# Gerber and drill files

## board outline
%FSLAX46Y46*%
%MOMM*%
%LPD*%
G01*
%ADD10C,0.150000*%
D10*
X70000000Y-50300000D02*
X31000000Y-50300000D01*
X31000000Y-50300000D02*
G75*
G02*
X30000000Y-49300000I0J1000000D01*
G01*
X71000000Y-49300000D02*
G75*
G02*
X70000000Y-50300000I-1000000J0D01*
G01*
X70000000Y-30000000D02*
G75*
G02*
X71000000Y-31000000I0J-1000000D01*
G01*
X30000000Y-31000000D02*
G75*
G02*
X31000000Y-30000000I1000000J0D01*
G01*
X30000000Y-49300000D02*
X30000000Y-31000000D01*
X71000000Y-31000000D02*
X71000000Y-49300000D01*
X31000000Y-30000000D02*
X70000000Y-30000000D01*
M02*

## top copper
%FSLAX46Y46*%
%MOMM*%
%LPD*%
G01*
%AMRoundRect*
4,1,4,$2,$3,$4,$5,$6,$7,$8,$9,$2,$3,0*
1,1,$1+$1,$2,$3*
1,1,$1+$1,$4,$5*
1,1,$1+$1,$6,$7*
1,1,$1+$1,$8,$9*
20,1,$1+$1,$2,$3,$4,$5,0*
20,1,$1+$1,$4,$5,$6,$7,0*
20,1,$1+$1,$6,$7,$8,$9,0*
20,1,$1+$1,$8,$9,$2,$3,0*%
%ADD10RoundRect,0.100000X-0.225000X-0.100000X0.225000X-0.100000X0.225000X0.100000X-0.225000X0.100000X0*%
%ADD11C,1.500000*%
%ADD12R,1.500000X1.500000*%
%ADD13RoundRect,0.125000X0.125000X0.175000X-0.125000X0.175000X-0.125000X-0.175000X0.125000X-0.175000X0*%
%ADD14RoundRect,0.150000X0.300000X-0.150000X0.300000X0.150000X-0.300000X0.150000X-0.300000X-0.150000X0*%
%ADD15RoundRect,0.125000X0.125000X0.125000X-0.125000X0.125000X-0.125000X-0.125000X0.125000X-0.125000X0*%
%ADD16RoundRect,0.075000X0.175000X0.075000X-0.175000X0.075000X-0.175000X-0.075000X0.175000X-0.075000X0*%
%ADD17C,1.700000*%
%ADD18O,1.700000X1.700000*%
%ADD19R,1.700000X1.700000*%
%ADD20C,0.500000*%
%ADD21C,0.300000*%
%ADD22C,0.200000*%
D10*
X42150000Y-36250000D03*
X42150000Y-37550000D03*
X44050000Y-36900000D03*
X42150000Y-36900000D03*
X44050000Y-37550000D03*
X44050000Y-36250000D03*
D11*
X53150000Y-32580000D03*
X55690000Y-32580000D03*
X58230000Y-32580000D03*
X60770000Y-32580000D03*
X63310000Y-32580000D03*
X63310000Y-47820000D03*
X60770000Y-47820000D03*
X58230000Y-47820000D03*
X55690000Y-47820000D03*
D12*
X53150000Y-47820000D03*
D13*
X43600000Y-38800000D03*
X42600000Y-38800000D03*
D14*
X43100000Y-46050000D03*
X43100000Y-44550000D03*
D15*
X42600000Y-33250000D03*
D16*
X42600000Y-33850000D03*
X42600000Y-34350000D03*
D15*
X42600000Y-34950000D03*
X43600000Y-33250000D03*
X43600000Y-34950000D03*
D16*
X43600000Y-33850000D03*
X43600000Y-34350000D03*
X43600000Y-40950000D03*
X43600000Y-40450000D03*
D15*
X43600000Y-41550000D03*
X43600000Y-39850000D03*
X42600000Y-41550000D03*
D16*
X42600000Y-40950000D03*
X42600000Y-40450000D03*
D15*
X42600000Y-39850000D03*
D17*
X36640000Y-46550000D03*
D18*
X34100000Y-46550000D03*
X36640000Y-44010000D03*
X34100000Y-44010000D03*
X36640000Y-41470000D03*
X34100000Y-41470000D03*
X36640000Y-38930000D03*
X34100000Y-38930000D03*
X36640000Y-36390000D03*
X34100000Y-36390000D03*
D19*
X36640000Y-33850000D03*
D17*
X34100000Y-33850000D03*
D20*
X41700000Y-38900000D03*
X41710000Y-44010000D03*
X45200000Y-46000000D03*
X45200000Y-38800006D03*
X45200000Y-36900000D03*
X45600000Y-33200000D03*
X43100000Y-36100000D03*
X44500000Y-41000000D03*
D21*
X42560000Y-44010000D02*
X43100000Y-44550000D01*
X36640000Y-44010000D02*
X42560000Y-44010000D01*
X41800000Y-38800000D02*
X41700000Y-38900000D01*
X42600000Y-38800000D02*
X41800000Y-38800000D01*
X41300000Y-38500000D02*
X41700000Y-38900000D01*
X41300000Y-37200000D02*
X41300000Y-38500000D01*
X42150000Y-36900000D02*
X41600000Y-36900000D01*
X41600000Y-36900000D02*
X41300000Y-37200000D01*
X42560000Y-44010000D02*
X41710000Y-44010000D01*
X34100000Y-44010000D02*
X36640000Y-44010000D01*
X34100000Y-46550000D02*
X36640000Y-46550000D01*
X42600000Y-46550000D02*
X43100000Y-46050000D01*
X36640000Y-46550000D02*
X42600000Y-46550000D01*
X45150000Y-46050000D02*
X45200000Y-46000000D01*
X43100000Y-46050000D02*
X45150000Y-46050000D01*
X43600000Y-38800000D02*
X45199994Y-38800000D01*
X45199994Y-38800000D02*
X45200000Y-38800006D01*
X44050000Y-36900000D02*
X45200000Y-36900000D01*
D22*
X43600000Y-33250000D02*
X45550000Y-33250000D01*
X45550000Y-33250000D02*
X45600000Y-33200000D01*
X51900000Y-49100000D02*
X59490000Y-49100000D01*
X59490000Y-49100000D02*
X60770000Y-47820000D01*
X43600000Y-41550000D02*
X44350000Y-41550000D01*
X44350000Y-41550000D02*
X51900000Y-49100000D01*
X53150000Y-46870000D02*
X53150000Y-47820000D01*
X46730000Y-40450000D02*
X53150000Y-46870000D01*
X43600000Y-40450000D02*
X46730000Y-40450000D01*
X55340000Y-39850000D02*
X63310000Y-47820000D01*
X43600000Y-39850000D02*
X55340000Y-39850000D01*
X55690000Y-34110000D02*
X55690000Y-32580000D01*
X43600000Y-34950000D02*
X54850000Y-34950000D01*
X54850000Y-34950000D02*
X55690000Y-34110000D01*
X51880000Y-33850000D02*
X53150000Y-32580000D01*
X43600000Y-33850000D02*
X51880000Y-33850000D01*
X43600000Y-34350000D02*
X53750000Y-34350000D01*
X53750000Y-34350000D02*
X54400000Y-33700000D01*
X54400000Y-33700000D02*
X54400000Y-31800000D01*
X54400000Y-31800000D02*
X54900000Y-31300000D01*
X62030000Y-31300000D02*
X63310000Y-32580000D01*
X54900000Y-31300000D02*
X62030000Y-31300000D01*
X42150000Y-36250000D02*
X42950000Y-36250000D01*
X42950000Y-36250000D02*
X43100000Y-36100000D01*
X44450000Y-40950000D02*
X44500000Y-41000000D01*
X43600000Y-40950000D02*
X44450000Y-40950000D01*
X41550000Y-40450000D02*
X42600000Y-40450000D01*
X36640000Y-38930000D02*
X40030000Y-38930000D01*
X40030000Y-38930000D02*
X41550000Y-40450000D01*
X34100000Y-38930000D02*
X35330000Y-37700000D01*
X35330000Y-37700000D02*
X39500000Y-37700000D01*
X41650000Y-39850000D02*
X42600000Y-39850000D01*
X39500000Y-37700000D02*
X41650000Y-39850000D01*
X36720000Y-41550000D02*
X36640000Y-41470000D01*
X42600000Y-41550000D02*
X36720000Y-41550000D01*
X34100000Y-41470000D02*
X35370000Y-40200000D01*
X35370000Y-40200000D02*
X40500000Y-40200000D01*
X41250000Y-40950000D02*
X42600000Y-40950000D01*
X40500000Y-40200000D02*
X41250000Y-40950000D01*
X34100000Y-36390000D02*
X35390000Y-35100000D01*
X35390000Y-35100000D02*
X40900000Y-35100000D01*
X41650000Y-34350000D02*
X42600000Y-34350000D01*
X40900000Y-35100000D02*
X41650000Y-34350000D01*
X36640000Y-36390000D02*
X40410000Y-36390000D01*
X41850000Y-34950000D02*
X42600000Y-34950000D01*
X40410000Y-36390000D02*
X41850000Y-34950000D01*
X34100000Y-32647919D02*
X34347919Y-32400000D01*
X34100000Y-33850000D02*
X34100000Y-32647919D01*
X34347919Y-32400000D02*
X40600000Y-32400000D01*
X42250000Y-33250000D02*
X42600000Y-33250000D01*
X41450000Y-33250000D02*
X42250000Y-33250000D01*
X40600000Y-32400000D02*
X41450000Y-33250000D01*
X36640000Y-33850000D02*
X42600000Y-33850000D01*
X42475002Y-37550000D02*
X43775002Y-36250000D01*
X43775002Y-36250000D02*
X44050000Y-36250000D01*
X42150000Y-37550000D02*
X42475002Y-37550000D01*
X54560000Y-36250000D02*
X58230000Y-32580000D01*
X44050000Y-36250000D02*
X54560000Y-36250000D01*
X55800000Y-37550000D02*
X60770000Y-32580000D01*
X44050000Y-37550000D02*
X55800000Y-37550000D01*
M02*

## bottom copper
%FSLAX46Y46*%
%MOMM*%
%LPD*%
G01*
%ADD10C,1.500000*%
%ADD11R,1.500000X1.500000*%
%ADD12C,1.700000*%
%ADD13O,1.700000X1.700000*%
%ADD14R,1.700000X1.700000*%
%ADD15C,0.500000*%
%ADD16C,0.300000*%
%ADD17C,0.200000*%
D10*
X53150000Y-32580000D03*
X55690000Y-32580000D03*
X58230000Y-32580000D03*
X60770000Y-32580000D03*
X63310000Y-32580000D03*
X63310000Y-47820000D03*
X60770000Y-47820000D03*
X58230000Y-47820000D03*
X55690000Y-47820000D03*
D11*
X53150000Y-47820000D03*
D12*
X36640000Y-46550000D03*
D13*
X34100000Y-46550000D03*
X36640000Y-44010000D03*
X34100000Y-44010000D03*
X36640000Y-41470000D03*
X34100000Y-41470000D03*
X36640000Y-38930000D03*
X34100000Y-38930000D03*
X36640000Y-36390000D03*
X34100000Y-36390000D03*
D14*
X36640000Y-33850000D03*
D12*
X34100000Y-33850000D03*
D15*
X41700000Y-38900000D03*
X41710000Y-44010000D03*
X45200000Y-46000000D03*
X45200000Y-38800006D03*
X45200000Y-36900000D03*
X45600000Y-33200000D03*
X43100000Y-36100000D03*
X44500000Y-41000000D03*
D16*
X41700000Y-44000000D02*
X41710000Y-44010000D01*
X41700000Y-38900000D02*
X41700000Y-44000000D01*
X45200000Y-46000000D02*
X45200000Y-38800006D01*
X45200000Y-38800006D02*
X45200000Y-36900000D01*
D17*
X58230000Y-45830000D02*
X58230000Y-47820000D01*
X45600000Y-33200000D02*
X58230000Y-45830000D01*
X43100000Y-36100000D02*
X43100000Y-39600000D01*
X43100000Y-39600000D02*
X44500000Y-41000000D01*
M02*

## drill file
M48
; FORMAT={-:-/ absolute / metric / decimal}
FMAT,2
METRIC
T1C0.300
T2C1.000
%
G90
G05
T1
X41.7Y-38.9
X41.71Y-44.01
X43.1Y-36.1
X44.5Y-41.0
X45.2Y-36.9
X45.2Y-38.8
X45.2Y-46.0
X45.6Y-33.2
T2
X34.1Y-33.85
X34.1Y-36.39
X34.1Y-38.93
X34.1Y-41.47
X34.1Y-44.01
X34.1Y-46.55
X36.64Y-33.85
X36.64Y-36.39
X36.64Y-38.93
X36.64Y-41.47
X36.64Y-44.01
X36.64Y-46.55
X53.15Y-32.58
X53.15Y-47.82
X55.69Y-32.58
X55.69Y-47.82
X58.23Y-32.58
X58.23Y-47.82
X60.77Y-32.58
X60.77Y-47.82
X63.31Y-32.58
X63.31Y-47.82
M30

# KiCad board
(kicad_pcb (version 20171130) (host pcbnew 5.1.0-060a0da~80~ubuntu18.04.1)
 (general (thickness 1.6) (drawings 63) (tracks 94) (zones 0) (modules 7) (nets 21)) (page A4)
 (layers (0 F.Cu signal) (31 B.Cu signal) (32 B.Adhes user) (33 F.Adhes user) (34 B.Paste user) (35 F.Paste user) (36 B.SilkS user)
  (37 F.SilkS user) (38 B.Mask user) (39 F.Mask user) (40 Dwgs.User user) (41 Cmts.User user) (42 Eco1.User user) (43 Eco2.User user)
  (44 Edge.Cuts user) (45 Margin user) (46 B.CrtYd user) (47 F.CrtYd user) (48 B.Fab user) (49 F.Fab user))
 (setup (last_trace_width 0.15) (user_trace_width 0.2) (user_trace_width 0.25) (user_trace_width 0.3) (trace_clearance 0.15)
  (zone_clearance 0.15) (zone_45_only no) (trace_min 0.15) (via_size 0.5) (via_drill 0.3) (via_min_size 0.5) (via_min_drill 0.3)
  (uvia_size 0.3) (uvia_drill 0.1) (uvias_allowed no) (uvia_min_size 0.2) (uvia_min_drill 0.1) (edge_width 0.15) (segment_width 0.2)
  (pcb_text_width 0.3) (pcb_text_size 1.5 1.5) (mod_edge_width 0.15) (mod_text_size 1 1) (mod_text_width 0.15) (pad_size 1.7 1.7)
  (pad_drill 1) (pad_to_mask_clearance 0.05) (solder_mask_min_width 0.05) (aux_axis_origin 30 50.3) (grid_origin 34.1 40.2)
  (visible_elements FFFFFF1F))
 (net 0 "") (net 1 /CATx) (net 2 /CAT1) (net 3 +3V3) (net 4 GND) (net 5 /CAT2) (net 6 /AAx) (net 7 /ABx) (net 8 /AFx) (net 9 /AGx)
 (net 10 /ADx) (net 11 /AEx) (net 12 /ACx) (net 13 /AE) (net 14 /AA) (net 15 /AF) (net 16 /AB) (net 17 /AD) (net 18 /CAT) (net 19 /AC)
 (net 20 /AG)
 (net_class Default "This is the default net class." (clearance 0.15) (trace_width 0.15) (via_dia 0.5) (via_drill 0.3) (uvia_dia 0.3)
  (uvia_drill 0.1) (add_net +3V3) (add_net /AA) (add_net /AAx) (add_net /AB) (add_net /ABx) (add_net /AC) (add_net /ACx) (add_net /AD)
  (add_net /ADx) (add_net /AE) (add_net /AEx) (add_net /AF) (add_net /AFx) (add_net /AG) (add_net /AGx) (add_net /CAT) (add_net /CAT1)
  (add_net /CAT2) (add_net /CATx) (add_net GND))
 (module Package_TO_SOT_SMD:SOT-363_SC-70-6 (layer F.Cu) (at 43.1 36.9)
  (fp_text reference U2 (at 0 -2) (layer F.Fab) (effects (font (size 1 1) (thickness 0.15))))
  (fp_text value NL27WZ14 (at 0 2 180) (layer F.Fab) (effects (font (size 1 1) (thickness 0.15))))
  (pad 1 smd roundrect (at -0.95 -0.65) (size 0.65 0.4) (layers F.Cu F.Paste F.Mask) (roundrect_rratio 0.25) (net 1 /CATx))
  (pad 3 smd roundrect (at -0.95 0.65) (size 0.65 0.4) (layers F.Cu F.Paste F.Mask) (roundrect_rratio 0.25) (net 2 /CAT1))
  (pad 5 smd roundrect (at 0.95 0) (size 0.65 0.4) (layers F.Cu F.Paste F.Mask) (roundrect_rratio 0.25) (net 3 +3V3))
  (pad 2 smd roundrect (at -0.95 0) (size 0.65 0.4) (layers F.Cu F.Paste F.Mask) (roundrect_rratio 0.25) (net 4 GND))
  (pad 4 smd roundrect (at 0.95 0.65) (size 0.65 0.4) (layers F.Cu F.Paste F.Mask) (roundrect_rratio 0.25) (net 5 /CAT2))
  (pad 6 smd roundrect (at 0.95 -0.65) (size 0.65 0.4) (layers F.Cu F.Paste F.Mask) (roundrect_rratio 0.25) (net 2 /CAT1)))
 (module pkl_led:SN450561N (layer F.Cu) (at 53.15 47.82 90)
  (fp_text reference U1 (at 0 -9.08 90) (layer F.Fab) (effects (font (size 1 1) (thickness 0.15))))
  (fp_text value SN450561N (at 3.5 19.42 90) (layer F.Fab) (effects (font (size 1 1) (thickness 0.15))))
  (pad 10 thru_hole circle (at 15.24 0 90) (size 1.5 1.5) (drill 1) (layers *.Cu *.Mask) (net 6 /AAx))
  (pad 9 thru_hole circle (at 15.24 2.54 90) (size 1.5 1.5) (drill 1) (layers *.Cu *.Mask) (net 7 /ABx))
  (pad 8 thru_hole circle (at 15.24 5.08 90) (size 1.5 1.5) (drill 1) (layers *.Cu *.Mask) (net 2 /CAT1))
  (pad 7 thru_hole circle (at 15.24 7.62 90) (size 1.5 1.5) (drill 1) (layers *.Cu *.Mask) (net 5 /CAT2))
  (pad 6 thru_hole circle (at 15.24 10.16 90) (size 1.5 1.5) (drill 1) (layers *.Cu *.Mask) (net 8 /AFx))
  (pad 5 thru_hole circle (at 0 10.16 90) (size 1.5 1.5) (drill 1) (layers *.Cu *.Mask) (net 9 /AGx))
  (pad 4 thru_hole circle (at 0 7.62 90) (size 1.5 1.5) (drill 1) (layers *.Cu *.Mask) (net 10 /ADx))
  (pad 3 thru_hole circle (at 0 5.08 90) (size 1.5 1.5) (drill 1) (layers *.Cu *.Mask) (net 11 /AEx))
  (pad 2 thru_hole circle (at 0 2.54 90) (size 1.5 1.5) (drill 1) (layers *.Cu *.Mask))
  (pad 1 thru_hole rect (at 0 0 90) (size 1.5 1.5) (drill 1) (layers *.Cu *.Mask) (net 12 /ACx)))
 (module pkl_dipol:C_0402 (layer F.Cu) (at 43.1 38.8 180)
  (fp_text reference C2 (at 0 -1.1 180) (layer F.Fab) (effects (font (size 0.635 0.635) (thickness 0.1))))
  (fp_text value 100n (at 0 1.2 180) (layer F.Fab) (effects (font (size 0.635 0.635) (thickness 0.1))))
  (pad 1 smd roundrect (at -0.5 0 180) (size 0.5 0.6) (layers F.Cu F.Paste F.Mask) (roundrect_rratio 0.25) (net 3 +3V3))
  (pad 2 smd roundrect (at 0.5 0 180) (size 0.5 0.6) (layers F.Cu F.Paste F.Mask) (roundrect_rratio 0.25) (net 4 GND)))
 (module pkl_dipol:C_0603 (layer F.Cu) (at 43.1 45.3 90)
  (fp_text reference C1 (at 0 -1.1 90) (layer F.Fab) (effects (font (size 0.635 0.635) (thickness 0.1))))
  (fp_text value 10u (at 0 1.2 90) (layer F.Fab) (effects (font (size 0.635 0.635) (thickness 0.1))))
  (pad 1 smd roundrect (at -0.75 0 90) (size 0.6 0.9) (layers F.Cu F.Paste F.Mask) (roundrect_rratio 0.25) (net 3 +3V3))
  (pad 2 smd roundrect (at 0.75 0 90) (size 0.6 0.9) (layers F.Cu F.Paste F.Mask) (roundrect_rratio 0.25) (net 4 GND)))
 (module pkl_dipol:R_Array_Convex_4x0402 (layer F.Cu) (at 43.1 34.1 180) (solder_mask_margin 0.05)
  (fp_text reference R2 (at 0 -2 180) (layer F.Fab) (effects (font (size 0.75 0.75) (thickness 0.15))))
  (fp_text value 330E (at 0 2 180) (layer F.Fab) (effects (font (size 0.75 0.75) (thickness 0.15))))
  (pad 8 smd roundrect (at 0.5 0.85 180) (size 0.5 0.5) (layers F.Cu F.Paste F.Mask) (roundrect_rratio 0.25) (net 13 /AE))
  (pad 6 smd roundrect (at 0.5 0.25 180) (size 0.5 0.3) (layers F.Cu F.Paste F.Mask) (roundrect_rratio 0.25) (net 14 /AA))
  (pad 4 smd roundrect (at 0.5 -0.25 180) (size 0.5 0.3) (layers F.Cu F.Paste F.Mask) (roundrect_rratio 0.25) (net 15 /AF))
  (pad 2 smd roundrect (at 0.5 -0.85 180) (size 0.5 0.5) (layers F.Cu F.Paste F.Mask) (roundrect_rratio 0.25) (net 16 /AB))
  (pad 7 smd roundrect (at -0.5 0.85 180) (size 0.5 0.5) (layers F.Cu F.Paste F.Mask) (roundrect_rratio 0.25) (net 11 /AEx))
  (pad 1 smd roundrect (at -0.5 -0.85 180) (size 0.5 0.5) (layers F.Cu F.Paste F.Mask) (roundrect_rratio 0.25) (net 7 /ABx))
  (pad 5 smd roundrect (at -0.5 0.25 180) (size 0.5 0.3) (layers F.Cu F.Paste F.Mask) (roundrect_rratio 0.25) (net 6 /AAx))
  (pad 3 smd roundrect (at -0.5 -0.25 180) (size 0.5 0.3) (layers F.Cu F.Paste F.Mask) (roundrect_rratio 0.25) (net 8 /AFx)))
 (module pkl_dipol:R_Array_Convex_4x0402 (layer F.Cu) (at 43.1 40.7 180) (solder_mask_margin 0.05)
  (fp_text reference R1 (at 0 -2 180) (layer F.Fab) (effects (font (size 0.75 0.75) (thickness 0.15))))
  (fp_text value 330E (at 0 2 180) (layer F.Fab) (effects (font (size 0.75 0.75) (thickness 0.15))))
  (pad 3 smd roundrect (at -0.5 -0.25 180) (size 0.5 0.3) (layers F.Cu F.Paste F.Mask) (roundrect_rratio 0.25) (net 1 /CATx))
  (pad 5 smd roundrect (at -0.5 0.25 180) (size 0.5 0.3) (layers F.Cu F.Paste F.Mask) (roundrect_rratio 0.25) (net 12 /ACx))
  (pad 1 smd roundrect (at -0.5 -0.85 180) (size 0.5 0.5) (layers F.Cu F.Paste F.Mask) (roundrect_rratio 0.25) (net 10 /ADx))
  (pad 7 smd roundrect (at -0.5 0.85 180) (size 0.5 0.5) (layers F.Cu F.Paste F.Mask) (roundrect_rratio 0.25) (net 9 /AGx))
  (pad 2 smd roundrect (at 0.5 -0.85 180) (size 0.5 0.5) (layers F.Cu F.Paste F.Mask) (roundrect_rratio 0.25) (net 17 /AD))
  (pad 4 smd roundrect (at 0.5 -0.25 180) (size 0.5 0.3) (layers F.Cu F.Paste F.Mask) (roundrect_rratio 0.25) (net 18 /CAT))
  (pad 6 smd roundrect (at 0.5 0.25 180) (size 0.5 0.3) (layers F.Cu F.Paste F.Mask) (roundrect_rratio 0.25) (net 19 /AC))
  (pad 8 smd roundrect (at 0.5 0.85 180) (size 0.5 0.5) (layers F.Cu F.Paste F.Mask) (roundrect_rratio 0.25) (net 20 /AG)))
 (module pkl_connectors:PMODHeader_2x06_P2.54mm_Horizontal (layer F.Cu) (at 36.64 46.55 180)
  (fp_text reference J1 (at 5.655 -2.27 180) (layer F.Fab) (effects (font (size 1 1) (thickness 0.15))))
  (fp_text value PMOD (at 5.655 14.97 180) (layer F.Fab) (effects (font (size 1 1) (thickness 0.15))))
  (pad 6 thru_hole circle (at 0 0 180) (size 1.7 1.7) (drill 1) (layers *.Cu *.Mask) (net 3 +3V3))
  (pad 12 thru_hole oval (at 2.54 0 180) (size 1.7 1.7) (drill 1) (layers *.Cu *.Mask) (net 3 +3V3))
  (pad 5 thru_hole oval (at 0 2.54 180) (size 1.7 1.7) (drill 1) (layers *.Cu *.Mask) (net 4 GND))
  (pad 11 thru_hole oval (at 2.54 2.54 180) (size 1.7 1.7) (drill 1) (layers *.Cu *.Mask) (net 4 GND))
  (pad 4 thru_hole oval (at 0 5.08 180) (size 1.7 1.7) (drill 1) (layers *.Cu *.Mask) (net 17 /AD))
  (pad 10 thru_hole oval (at 2.54 5.08 180) (size 1.7 1.7) (drill 1) (layers *.Cu *.Mask) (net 18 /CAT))
  (pad 3 thru_hole oval (at 0 7.62 180) (size 1.7 1.7) (drill 1) (layers *.Cu *.Mask) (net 19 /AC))
  (pad 9 thru_hole oval (at 2.54 7.62 180) (size 1.7 1.7) (drill 1) (layers *.Cu *.Mask) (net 20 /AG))
  (pad 2 thru_hole oval (at 0 10.16 180) (size 1.7 1.7) (drill 1) (layers *.Cu *.Mask) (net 16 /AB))
  (pad 8 thru_hole oval (at 2.54 10.16 180) (size 1.7 1.7) (drill 1) (layers *.Cu *.Mask) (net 15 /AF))
  (pad 1 thru_hole rect (at 0 12.7 180) (size 1.7 1.7) (drill 1) (layers *.Cu *.Mask) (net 14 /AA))
  (pad 7 thru_hole circle (at 2.54 12.7 180) (size 1.7 1.7) (drill 1) (layers *.Cu *.Mask) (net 13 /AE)))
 (gr_line (start 70 50.3) (end 31 50.3) (layer Edge.Cuts) (width 0.15))
 (gr_arc (start 31 49.3) (end 30 49.3) (angle -90) (layer Edge.Cuts) (width 0.15))
 (gr_arc (start 70 49.3) (end 70 50.3) (angle -90) (layer Edge.Cuts) (width 0.15))
 (gr_arc (start 70 31) (end 71 31) (angle -90) (layer Edge.Cuts) (width 0.15))
 (gr_arc (start 31 31) (end 31 30) (angle -90) (layer Edge.Cuts) (width 0.15))
 (gr_line (start 30 49.3) (end 30 31) (layer Edge.Cuts) (width 0.15))
 (gr_line (start 71 31) (end 71 49.3) (layer Edge.Cuts) (width 0.15))
 (gr_line (start 31 30) (end 70 30) (layer Edge.Cuts) (width 0.15))
 (segment (start 42.56 44.01) (end 43.1 44.55) (width 0.3) (layer F.Cu) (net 4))
 (segment (start 36.64 44.01) (end 42.56 44.01) (width 0.3) (layer F.Cu) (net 4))
 (via (at 41.7 38.9) (size 0.5) (drill 0.3) (layers F.Cu B.Cu) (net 4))
 (segment (start 41.8 38.8) (end 41.7 38.9) (width 0.3) (layer F.Cu) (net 4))
 (segment (start 42.6 38.8) (end 41.8 38.8) (width 0.3) (layer F.Cu) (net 4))
 (segment (start 41.3 38.5) (end 41.7 38.9) (width 0.3) (layer F.Cu) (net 4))
 (segment (start 41.3 37.2) (end 41.3 38.5) (width 0.3) (layer F.Cu) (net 4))
 (segment (start 42.15 36.9) (end 41.6 36.9) (width 0.3) (layer F.Cu) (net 4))
 (segment (start 41.6 36.9) (end 41.3 37.2) (width 0.3) (layer F.Cu) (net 4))
 (segment (start 42.56 44.01) (end 41.71 44.01) (width 0.3) (layer F.Cu) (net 4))
 (segment (start 41.7 44) (end 41.71 44.01) (width 0.3) (layer B.Cu) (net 4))
 (via (at 41.71 44.01) (size 0.5) (drill 0.3) (layers F.Cu B.Cu) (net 4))
 (segment (start 41.7 38.9) (end 41.7 44) (width 0.3) (layer B.Cu) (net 4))
 (segment (start 34.1 44.01) (end 36.64 44.01) (width 0.3) (layer F.Cu) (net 4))
 (segment (start 34.1 46.55) (end 36.64 46.55) (width 0.3) (layer F.Cu) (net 3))
 (segment (start 42.6 46.55) (end 43.1 46.05) (width 0.3) (layer F.Cu) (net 3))
 (segment (start 36.64 46.55) (end 42.6 46.55) (width 0.3) (layer F.Cu) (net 3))
 (segment (start 45.15 46.05) (end 45.2 46) (width 0.3) (layer F.Cu) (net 3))
 (via (at 45.2 46) (size 0.5) (drill 0.3) (layers F.Cu B.Cu) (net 3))
 (segment (start 43.1 46.05) (end 45.15 46.05) (width 0.3) (layer F.Cu) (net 3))
 (via (at 45.2 38.800006) (size 0.5) (drill 0.3) (layers F.Cu B.Cu) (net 3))
 (segment (start 43.6 38.8) (end 45.199994 38.8) (width 0.3) (layer F.Cu) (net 3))
 (segment (start 45.199994 38.8) (end 45.2 38.800006) (width 0.3) (layer F.Cu) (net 3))
 (segment (start 45.2 46) (end 45.2 38.800006) (width 0.3) (layer B.Cu) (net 3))
 (via (at 45.2 36.9) (size 0.5) (drill 0.3) (layers F.Cu B.Cu) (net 3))
 (segment (start 45.2 38.800006) (end 45.2 36.9) (width 0.3) (layer B.Cu) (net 3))
 (segment (start 44.05 36.9) (end 45.2 36.9) (width 0.3) (layer F.Cu) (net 3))
 (via (at 45.6 33.2) (size 0.5) (drill 0.3) (layers F.Cu B.Cu) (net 11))
 (segment (start 43.6 33.25) (end 45.55 33.25) (width 0.2) (layer F.Cu) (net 11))
 (segment (start 45.55 33.25) (end 45.6 33.2) (width 0.2) (layer F.Cu) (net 11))
 (segment (start 58.23 45.83) (end 58.23 47.82) (width 0.2) (layer B.Cu) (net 11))
 (segment (start 45.6 33.2) (end 58.23 45.83) (width 0.2) (layer B.Cu) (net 11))
 (segment (start 51.9 49.1) (end 59.49 49.1) (width 0.2) (layer F.Cu) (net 10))
 (segment (start 59.49 49.1) (end 60.77 47.82) (width 0.2) (layer F.Cu) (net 10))
 (segment (start 43.6 41.55) (end 44.35 41.55) (width 0.2) (layer F.Cu) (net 10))
 (segment (start 44.35 41.55) (end 51.9 49.1) (width 0.2) (layer F.Cu) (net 10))
 (segment (start 53.15 46.87) (end 53.15 47.82) (width 0.2) (layer F.Cu) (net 12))
 (segment (start 46.73 40.45) (end 53.15 46.87) (width 0.2) (layer F.Cu) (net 12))
 (segment (start 43.6 40.45) (end 46.73 40.45) (width 0.2) (layer F.Cu) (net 12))
 (segment (start 55.34 39.85) (end 63.31 47.82) (width 0.2) (layer F.Cu) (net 9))
 (segment (start 43.6 39.85) (end 55.34 39.85) (width 0.2) (layer F.Cu) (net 9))
 (segment (start 55.69 34.11) (end 55.69 32.58) (width 0.2) (layer F.Cu) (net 7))
 (segment (start 43.6 34.95) (end 54.85 34.95) (width 0.2) (layer F.Cu) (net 7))
 (segment (start 54.85 34.95) (end 55.69 34.11) (width 0.2) (layer F.Cu) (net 7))
 (segment (start 51.88 33.85) (end 53.15 32.58) (width 0.2) (layer F.Cu) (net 6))
 (segment (start 43.6 33.85) (end 51.88 33.85) (width 0.2) (layer F.Cu) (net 6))
 (segment (start 43.6 34.35) (end 53.75 34.35) (width 0.2) (layer F.Cu) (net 8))
 (segment (start 53.75 34.35) (end 54.4 33.7) (width 0.2) (layer F.Cu) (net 8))
 (segment (start 54.4 33.7) (end 54.4 31.8) (width 0.2) (layer F.Cu) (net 8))
 (segment (start 54.4 31.8) (end 54.9 31.3) (width 0.2) (layer F.Cu) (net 8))
 (segment (start 62.03 31.3) (end 63.31 32.58) (width 0.2) (layer F.Cu) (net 8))
 (segment (start 54.9 31.3) (end 62.03 31.3) (width 0.2) (layer F.Cu) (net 8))
 (via (at 43.1 36.1) (size 0.5) (drill 0.3) (layers F.Cu B.Cu) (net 1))
 (segment (start 42.15 36.25) (end 42.95 36.25) (width 0.2) (layer F.Cu) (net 1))
 (segment (start 42.95 36.25) (end 43.1 36.1) (width 0.2) (layer F.Cu) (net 1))
 (via (at 44.5 41) (size 0.5) (drill 0.3) (layers F.Cu B.Cu) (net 1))
 (segment (start 43.1 36.1) (end 43.1 39.6) (width 0.2) (layer B.Cu) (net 1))
 (segment (start 43.1 39.6) (end 44.5 41) (width 0.2) (layer B.Cu) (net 1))
 (segment (start 44.45 40.95) (end 44.5 41) (width 0.2) (layer F.Cu) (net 1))
 (segment (start 43.6 40.95) (end 44.45 40.95) (width 0.2) (layer F.Cu) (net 1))
 (segment (start 41.55 40.45) (end 42.6 40.45) (width 0.2) (layer F.Cu) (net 19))
 (segment (start 36.64 38.93) (end 40.03 38.93) (width 0.2) (layer F.Cu) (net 19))
 (segment (start 40.03 38.93) (end 41.55 40.45) (width 0.2) (layer F.Cu) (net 19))
 (segment (start 34.1 38.93) (end 35.33 37.7) (width 0.2) (layer F.Cu) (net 20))
 (segment (start 35.33 37.7) (end 39.5 37.7) (width 0.2) (layer F.Cu) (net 20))
 (segment (start 41.65 39.85) (end 42.6 39.85) (width 0.2) (layer F.Cu) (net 20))
 (segment (start 39.5 37.7) (end 41.65 39.85) (width 0.2) (layer F.Cu) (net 20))
 (segment (start 36.72 41.55) (end 36.64 41.47) (width 0.2) (layer F.Cu) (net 17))
 (segment (start 42.6 41.55) (end 36.72 41.55) (width 0.2) (layer F.Cu) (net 17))
 (segment (start 34.1 41.47) (end 35.37 40.2) (width 0.2) (layer F.Cu) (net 18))
 (segment (start 35.37 40.2) (end 40.5 40.2) (width 0.2) (layer F.Cu) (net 18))
 (segment (start 41.25 40.95) (end 42.6 40.95) (width 0.2) (layer F.Cu) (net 18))
 (segment (start 40.5 40.2) (end 41.25 40.95) (width 0.2) (layer F.Cu) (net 18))
 (segment (start 34.1 36.39) (end 35.39 35.1) (width 0.2) (layer F.Cu) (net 15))
 (segment (start 35.39 35.1) (end 40.9 35.1) (width 0.2) (layer F.Cu) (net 15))
 (segment (start 41.65 34.35) (end 42.6 34.35) (width 0.2) (layer F.Cu) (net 15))
 (segment (start 40.9 35.1) (end 41.65 34.35) (width 0.2) (layer F.Cu) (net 15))
 (segment (start 36.64 36.39) (end 40.41 36.39) (width 0.2) (layer F.Cu) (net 16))
 (segment (start 41.85 34.95) (end 42.6 34.95) (width 0.2) (layer F.Cu) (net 16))
 (segment (start 40.41 36.39) (end 41.85 34.95) (width 0.2) (layer F.Cu) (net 16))
 (segment (start 34.1 32.647919) (end 34.347919 32.4) (width 0.2) (layer F.Cu) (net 13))
 (segment (start 34.1 33.85) (end 34.1 32.647919) (width 0.2) (layer F.Cu) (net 13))
 (segment (start 34.347919 32.4) (end 40.6 32.4) (width 0.2) (layer F.Cu) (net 13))
 (segment (start 42.25 33.25) (end 42.6 33.25) (width 0.2) (layer F.Cu) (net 13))
 (segment (start 41.45 33.25) (end 42.25 33.25) (width 0.2) (layer F.Cu) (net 13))
 (segment (start 40.6 32.4) (end 41.45 33.25) (width 0.2) (layer F.Cu) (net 13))
 (segment (start 36.64 33.85) (end 42.6 33.85) (width 0.2) (layer F.Cu) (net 14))
 (segment (start 42.475002 37.55) (end 43.775002 36.25) (width 0.2) (layer F.Cu) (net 2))
 (segment (start 43.775002 36.25) (end 44.05 36.25) (width 0.2) (layer F.Cu) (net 2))
 (segment (start 42.15 37.55) (end 42.475002 37.55) (width 0.2) (layer F.Cu) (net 2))
 (segment (start 54.56 36.25) (end 58.23 32.58) (width 0.2) (layer F.Cu) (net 2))
 (segment (start 44.05 36.25) (end 54.56 36.25) (width 0.2) (layer F.Cu) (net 2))
 (segment (start 55.8 37.55) (end 60.77 32.58) (width 0.2) (layer F.Cu) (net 5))
 (segment (start 44.05 37.55) (end 55.8 37.55) (width 0.2) (layer F.Cu) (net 5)))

